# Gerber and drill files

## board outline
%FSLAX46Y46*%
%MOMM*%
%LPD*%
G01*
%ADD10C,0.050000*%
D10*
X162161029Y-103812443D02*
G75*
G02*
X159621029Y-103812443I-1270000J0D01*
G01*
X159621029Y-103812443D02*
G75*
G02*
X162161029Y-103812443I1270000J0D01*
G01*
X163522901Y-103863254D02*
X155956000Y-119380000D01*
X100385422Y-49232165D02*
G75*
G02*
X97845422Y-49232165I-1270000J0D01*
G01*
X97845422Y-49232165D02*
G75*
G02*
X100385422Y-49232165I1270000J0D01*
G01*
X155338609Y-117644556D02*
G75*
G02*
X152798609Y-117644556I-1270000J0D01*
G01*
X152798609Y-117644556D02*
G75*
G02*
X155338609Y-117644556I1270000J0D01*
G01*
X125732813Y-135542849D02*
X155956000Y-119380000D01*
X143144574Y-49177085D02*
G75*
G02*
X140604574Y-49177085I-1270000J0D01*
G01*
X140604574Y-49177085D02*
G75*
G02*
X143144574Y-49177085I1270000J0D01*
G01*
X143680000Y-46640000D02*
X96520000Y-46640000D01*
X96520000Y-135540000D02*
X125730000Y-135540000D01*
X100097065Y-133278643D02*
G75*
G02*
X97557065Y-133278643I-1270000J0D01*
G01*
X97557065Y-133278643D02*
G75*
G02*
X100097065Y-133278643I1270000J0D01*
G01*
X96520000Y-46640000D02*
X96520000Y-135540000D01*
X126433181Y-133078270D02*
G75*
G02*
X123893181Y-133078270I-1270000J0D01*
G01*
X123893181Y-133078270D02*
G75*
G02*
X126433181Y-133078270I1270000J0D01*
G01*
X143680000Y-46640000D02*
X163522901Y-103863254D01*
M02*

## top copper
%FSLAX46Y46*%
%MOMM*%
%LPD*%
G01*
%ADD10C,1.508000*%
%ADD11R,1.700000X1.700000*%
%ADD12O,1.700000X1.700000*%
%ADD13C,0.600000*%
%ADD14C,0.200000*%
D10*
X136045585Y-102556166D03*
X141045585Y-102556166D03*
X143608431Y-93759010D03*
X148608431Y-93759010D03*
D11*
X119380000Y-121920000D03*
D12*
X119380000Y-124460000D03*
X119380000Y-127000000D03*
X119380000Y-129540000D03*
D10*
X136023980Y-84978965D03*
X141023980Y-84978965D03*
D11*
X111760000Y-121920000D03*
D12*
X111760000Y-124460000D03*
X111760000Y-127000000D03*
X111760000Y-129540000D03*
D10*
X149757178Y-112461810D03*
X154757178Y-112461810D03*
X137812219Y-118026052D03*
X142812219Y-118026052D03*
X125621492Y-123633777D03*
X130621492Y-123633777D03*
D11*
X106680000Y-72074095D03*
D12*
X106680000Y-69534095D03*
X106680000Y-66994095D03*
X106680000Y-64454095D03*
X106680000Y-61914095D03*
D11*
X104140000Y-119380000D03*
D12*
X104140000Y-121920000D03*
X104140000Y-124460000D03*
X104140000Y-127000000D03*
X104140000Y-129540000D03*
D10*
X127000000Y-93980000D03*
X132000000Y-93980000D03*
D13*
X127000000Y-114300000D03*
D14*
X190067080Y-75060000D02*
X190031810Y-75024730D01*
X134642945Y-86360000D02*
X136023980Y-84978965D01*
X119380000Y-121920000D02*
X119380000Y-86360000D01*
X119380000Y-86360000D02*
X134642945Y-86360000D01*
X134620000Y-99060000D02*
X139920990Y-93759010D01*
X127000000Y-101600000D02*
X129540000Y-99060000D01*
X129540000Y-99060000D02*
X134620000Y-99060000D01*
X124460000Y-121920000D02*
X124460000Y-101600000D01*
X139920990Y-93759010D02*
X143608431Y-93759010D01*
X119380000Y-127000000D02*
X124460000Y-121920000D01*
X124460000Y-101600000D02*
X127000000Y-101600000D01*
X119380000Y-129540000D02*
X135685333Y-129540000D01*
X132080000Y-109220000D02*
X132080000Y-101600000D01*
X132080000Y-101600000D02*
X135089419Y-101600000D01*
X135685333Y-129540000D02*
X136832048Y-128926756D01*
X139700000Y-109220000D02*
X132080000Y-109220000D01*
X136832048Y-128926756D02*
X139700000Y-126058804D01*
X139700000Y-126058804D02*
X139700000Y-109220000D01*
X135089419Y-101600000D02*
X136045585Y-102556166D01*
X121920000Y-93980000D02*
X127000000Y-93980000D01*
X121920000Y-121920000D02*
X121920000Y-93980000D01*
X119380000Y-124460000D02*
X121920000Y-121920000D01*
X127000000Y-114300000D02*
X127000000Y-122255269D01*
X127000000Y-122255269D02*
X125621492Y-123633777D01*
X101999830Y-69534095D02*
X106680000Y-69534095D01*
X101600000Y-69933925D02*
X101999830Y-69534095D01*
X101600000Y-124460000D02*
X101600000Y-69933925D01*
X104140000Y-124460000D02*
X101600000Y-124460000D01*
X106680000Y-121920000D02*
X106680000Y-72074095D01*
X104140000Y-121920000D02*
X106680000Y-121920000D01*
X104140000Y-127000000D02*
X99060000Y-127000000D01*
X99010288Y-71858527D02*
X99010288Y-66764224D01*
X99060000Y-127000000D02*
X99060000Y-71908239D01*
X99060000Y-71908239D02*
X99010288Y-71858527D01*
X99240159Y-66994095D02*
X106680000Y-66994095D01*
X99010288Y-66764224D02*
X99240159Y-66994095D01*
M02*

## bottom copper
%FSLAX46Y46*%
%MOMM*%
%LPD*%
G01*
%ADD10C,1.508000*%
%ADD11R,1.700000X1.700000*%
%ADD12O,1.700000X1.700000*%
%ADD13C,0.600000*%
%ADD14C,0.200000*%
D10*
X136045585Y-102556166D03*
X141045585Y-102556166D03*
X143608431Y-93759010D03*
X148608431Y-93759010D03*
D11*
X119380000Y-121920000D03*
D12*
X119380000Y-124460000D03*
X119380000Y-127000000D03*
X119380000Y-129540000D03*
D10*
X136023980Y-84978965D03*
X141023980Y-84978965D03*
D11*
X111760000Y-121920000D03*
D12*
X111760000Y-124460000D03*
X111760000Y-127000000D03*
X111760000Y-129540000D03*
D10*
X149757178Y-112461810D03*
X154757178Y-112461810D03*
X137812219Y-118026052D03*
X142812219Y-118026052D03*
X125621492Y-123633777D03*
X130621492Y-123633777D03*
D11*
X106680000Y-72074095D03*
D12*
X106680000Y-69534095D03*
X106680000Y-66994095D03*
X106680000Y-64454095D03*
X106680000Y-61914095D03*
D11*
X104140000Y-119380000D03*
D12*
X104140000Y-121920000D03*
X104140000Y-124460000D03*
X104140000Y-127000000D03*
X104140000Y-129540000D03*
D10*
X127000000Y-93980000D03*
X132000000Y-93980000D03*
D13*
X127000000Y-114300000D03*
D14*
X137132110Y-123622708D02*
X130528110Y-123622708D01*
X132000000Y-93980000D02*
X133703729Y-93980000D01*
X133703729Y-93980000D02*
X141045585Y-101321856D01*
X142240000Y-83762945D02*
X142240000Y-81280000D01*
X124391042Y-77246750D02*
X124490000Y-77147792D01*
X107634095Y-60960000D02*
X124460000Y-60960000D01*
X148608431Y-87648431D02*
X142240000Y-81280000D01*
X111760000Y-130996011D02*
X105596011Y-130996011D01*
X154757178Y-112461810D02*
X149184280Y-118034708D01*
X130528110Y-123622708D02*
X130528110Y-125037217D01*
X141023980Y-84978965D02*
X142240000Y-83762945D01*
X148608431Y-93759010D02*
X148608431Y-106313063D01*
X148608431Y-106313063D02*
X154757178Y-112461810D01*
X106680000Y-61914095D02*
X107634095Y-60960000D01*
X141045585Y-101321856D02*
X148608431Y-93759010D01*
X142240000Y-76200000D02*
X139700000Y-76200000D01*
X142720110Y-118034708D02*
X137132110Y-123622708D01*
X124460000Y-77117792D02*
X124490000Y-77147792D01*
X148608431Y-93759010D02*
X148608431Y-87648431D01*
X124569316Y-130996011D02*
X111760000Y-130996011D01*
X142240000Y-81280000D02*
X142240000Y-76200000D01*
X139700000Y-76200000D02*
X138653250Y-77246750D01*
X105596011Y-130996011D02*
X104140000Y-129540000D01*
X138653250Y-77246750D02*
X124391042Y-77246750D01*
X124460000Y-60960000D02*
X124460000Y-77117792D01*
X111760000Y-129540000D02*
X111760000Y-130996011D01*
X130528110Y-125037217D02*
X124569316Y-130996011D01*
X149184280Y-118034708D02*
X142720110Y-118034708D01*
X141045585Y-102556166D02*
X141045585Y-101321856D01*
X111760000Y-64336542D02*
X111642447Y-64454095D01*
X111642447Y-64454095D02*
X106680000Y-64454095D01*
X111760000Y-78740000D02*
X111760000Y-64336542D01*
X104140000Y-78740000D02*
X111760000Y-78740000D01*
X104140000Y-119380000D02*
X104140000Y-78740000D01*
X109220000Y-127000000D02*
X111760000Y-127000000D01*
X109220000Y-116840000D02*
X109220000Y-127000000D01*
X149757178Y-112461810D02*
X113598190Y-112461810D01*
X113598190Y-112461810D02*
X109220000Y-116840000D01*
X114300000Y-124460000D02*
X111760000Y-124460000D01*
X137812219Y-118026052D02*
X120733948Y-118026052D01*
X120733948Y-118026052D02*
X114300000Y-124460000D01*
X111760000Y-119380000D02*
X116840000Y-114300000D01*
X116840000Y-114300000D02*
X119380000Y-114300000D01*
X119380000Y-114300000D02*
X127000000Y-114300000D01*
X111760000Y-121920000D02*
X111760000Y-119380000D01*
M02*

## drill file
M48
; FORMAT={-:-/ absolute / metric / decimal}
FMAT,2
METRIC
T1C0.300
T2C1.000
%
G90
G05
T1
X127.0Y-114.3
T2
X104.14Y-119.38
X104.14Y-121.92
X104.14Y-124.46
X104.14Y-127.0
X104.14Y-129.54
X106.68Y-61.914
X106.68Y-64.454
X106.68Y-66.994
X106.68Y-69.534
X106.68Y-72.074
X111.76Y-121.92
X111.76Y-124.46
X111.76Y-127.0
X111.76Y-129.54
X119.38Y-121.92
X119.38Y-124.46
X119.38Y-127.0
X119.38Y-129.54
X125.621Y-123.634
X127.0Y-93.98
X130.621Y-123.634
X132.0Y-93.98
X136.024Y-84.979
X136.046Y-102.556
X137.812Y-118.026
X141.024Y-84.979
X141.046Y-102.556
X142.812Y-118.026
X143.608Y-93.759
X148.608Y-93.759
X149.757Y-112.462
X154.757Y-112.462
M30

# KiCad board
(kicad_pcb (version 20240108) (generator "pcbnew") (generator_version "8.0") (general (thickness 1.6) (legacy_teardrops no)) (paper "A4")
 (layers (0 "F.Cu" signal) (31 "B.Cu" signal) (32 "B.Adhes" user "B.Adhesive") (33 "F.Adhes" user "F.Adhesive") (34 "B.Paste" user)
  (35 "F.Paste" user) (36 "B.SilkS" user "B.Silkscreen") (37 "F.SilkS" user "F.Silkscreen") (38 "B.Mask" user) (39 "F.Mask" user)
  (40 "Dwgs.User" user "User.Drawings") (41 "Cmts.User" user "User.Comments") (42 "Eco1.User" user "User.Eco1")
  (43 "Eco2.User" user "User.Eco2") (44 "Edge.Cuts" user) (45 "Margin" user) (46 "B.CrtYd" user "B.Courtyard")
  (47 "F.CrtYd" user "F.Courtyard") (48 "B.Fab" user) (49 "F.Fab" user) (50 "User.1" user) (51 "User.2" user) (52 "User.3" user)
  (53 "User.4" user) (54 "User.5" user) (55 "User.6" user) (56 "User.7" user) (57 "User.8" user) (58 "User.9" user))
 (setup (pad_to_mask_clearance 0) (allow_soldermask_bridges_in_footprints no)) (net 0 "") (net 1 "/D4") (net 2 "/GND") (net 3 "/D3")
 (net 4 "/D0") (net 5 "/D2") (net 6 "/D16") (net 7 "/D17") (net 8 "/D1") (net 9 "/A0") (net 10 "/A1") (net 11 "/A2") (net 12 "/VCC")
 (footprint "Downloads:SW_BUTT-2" (layer "F.Cu") (at 138.545585 102.556166)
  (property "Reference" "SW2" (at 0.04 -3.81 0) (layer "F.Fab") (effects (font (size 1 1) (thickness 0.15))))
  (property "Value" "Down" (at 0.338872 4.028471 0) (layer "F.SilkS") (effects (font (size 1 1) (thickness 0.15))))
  (pad "1" thru_hole circle (at -2.5 0) (size 1.508 1.508) (drill 1) (layers "*.Cu" "*.Mask") (remove_unused_layers no) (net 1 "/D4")
   (solder_mask_margin 0.102))
  (pad "2" thru_hole circle (at 2.5 0) (size 1.508 1.508) (drill 1) (layers "*.Cu" "*.Mask") (remove_unused_layers no) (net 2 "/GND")
   (solder_mask_margin 0.102)))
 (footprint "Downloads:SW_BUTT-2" (layer "F.Cu") (at 146.108431 93.75901)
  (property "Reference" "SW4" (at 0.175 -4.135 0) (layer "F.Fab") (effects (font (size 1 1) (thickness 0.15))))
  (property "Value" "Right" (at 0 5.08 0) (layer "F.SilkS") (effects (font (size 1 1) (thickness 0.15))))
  (pad "1" thru_hole circle (at -2.5 0) (size 1.508 1.508) (drill 1) (layers "*.Cu" "*.Mask") (remove_unused_layers no) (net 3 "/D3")
   (solder_mask_margin 0.102))
  (pad "2" thru_hole circle (at 2.5 0) (size 1.508 1.508) (drill 1) (layers "*.Cu" "*.Mask") (remove_unused_layers no) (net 2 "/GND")
   (solder_mask_margin 0.102)))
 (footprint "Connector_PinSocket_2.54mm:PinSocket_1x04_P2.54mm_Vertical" (layer "F.Cu") (at 119.38 121.92)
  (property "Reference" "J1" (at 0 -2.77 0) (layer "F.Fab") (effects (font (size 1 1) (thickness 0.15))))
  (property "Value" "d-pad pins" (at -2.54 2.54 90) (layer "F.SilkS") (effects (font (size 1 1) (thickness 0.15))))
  (pad "1" thru_hole rect (at 0 0) (size 1.7 1.7) (drill 1) (layers "*.Cu" "*.Mask") (remove_unused_layers no) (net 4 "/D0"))
  (pad "2" thru_hole oval (at 0 2.54) (size 1.7 1.7) (drill 1) (layers "*.Cu" "*.Mask") (remove_unused_layers no) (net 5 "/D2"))
  (pad "3" thru_hole oval (at 0 5.08) (size 1.7 1.7) (drill 1) (layers "*.Cu" "*.Mask") (remove_unused_layers no) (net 3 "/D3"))
  (pad "4" thru_hole oval (at 0 7.62) (size 1.7 1.7) (drill 1) (layers "*.Cu" "*.Mask") (remove_unused_layers no) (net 1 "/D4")))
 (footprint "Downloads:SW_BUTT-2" (layer "F.Cu") (at 138.52398 84.978965)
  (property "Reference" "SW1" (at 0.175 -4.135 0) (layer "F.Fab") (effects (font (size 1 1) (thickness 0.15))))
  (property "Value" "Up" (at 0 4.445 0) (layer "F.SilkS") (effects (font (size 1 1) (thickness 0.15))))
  (pad "1" thru_hole circle (at -2.5 0) (size 1.508 1.508) (drill 1) (layers "*.Cu" "*.Mask") (remove_unused_layers no) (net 4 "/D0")
   (solder_mask_margin 0.102))
  (pad "2" thru_hole circle (at 2.5 0) (size 1.508 1.508) (drill 1) (layers "*.Cu" "*.Mask") (remove_unused_layers no) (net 2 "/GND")
   (solder_mask_margin 0.102)))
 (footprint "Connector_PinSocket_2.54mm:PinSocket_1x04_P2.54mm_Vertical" (layer "F.Cu") (at 111.76 121.92)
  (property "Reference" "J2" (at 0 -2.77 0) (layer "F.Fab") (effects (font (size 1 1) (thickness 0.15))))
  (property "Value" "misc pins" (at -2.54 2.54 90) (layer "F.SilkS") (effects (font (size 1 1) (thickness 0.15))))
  (pad "1" thru_hole rect (at 0 0) (size 1.7 1.7) (drill 1) (layers "*.Cu" "*.Mask") (remove_unused_layers no) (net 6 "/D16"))
  (pad "2" thru_hole oval (at 0 2.54) (size 1.7 1.7) (drill 1) (layers "*.Cu" "*.Mask") (remove_unused_layers no) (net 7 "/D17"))
  (pad "3" thru_hole oval (at 0 5.08) (size 1.7 1.7) (drill 1) (layers "*.Cu" "*.Mask") (remove_unused_layers no) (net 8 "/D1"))
  (pad "4" thru_hole oval (at 0 7.62) (size 1.7 1.7) (drill 1) (layers "*.Cu" "*.Mask") (remove_unused_layers no) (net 2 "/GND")))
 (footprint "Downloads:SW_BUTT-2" (layer "F.Cu") (at 152.257178 112.46181)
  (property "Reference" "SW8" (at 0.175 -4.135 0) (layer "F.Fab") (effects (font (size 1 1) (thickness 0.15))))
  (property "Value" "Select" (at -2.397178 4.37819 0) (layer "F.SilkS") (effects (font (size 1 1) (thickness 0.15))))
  (pad "1" thru_hole circle (at -2.5 0) (size 1.508 1.508) (drill 1) (layers "*.Cu" "*.Mask") (remove_unused_layers no) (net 8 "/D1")
   (solder_mask_margin 0.102))
  (pad "2" thru_hole circle (at 2.5 0) (size 1.508 1.508) (drill 1) (layers "*.Cu" "*.Mask") (remove_unused_layers no) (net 2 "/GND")
   (solder_mask_margin 0.102)))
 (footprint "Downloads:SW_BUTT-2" (layer "F.Cu") (at 140.312219 118.026052)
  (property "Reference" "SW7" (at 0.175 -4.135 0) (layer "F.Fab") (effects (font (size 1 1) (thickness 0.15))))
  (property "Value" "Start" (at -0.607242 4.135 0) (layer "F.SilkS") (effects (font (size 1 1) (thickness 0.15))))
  (pad "1" thru_hole circle (at -2.5 0) (size 1.508 1.508) (drill 1) (layers "*.Cu" "*.Mask") (remove_unused_layers no) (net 7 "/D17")
   (solder_mask_margin 0.102))
  (pad "2" thru_hole circle (at 2.5 0) (size 1.508 1.508) (drill 1) (layers "*.Cu" "*.Mask") (remove_unused_layers no) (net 2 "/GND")
   (solder_mask_margin 0.102)))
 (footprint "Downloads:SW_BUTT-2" (layer "F.Cu") (at 128.121492 123.633777)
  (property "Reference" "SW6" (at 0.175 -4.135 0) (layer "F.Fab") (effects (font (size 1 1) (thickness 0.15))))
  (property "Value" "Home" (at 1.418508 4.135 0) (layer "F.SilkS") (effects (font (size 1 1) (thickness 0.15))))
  (pad "1" thru_hole circle (at -2.5 0) (size 1.508 1.508) (drill 1) (layers "*.Cu" "*.Mask") (remove_unused_layers no) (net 6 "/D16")
   (solder_mask_margin 0.102))
  (pad "2" thru_hole circle (at 2.5 0) (size 1.508 1.508) (drill 1) (layers "*.Cu" "*.Mask") (remove_unused_layers no) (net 2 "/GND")
   (solder_mask_margin 0.102)))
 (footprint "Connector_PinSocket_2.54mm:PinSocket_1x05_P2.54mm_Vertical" (layer "F.Cu") (at 106.68 72.074095 180)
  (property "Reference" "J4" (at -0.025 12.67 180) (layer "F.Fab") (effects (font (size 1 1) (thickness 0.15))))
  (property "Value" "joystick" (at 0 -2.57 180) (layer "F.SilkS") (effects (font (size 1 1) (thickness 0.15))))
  (pad "1" thru_hole rect (at 0 0 180) (size 1.7 1.7) (drill 1) (layers "*.Cu" "*.Mask") (remove_unused_layers no) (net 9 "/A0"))
  (pad "2" thru_hole oval (at 0 2.54 180) (size 1.7 1.7) (drill 1) (layers "*.Cu" "*.Mask") (remove_unused_layers no) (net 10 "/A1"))
  (pad "3" thru_hole oval (at 0 5.08 180) (size 1.7 1.7) (drill 1) (layers "*.Cu" "*.Mask") (remove_unused_layers no) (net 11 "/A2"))
  (pad "4" thru_hole oval (at 0 7.62 180) (size 1.7 1.7) (drill 1) (layers "*.Cu" "*.Mask") (remove_unused_layers no) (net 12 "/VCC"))
  (pad "5" thru_hole oval (at 0 10.16 180) (size 1.7 1.7) (drill 1) (layers "*.Cu" "*.Mask") (remove_unused_layers no) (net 2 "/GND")))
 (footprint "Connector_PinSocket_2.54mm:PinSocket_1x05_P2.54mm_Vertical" (layer "F.Cu") (at 104.14 119.38)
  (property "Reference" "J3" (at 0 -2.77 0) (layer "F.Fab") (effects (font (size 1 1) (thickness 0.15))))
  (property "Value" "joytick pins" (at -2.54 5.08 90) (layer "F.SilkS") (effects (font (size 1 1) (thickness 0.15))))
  (pad "1" thru_hole rect (at 0 0) (size 1.7 1.7) (drill 1) (layers "*.Cu" "*.Mask") (remove_unused_layers no) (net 12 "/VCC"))
  (pad "2" thru_hole oval (at 0 2.54) (size 1.7 1.7) (drill 1) (layers "*.Cu" "*.Mask") (remove_unused_layers no) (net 9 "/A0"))
  (pad "3" thru_hole oval (at 0 5.08) (size 1.7 1.7) (drill 1) (layers "*.Cu" "*.Mask") (remove_unused_layers no) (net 10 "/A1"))
  (pad "4" thru_hole oval (at 0 7.62) (size 1.7 1.7) (drill 1) (layers "*.Cu" "*.Mask") (remove_unused_layers no) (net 11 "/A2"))
  (pad "5" thru_hole oval (at 0 10.16) (size 1.7 1.7) (drill 1) (layers "*.Cu" "*.Mask") (remove_unused_layers no) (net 2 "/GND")))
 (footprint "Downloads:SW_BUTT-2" (layer "F.Cu") (at 129.5 93.98)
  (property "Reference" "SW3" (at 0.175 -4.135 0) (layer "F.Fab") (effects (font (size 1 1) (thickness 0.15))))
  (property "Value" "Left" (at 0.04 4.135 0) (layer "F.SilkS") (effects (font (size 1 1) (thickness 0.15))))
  (pad "1" thru_hole circle (at -2.5 0) (size 1.508 1.508) (drill 1) (layers "*.Cu" "*.Mask") (remove_unused_layers no) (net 5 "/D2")
   (solder_mask_margin 0.102))
  (pad "2" thru_hole circle (at 2.5 0) (size 1.508 1.508) (drill 1) (layers "*.Cu" "*.Mask") (remove_unused_layers no) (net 2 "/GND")
   (solder_mask_margin 0.102)))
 (gr_circle (center 160.891029 103.812443) (end 162.161029 103.812443) (stroke (width 0.05) (type default)) (fill none) (layer "Edge.Cuts"))
 (gr_line (start 163.522901 103.863254) (end 155.956 119.38) (stroke (width 0.05) (type default)) (layer "Edge.Cuts"))
 (gr_circle (center 99.115422 49.232165) (end 97.845422 49.232165) (stroke (width 0.05) (type default)) (fill none) (layer "Edge.Cuts"))
 (gr_circle (center 154.068609 117.644556) (end 155.338609 117.644556) (stroke (width 0.05) (type default)) (fill none) (layer "Edge.Cuts"))
 (gr_line (start 125.732813 135.542849) (end 155.956 119.38) (stroke (width 0.05) (type default)) (layer "Edge.Cuts"))
 (gr_circle (center 141.874574 49.177085) (end 141.874574 47.907085) (stroke (width 0.05) (type default)) (fill none) (layer "Edge.Cuts"))
 (gr_line (start 143.68 46.64) (end 96.52 46.64) (stroke (width 0.05) (type default)) (layer "Edge.Cuts"))
 (gr_line (start 96.52 135.54) (end 125.73 135.54) (stroke (width 0.05) (type default)) (layer "Edge.Cuts"))
 (gr_circle (center 98.827065 133.278643) (end 100.097065 133.278643) (stroke (width 0.05) (type default)) (fill none) (layer "Edge.Cuts"))
 (gr_line (start 96.52 46.64) (end 96.52 135.54) (stroke (width 0.05) (type default)) (layer "Edge.Cuts"))
 (gr_circle (center 125.163181 133.07827) (end 126.433181 133.07827) (stroke (width 0.05) (type default)) (fill none) (layer "Edge.Cuts"))
 (gr_line (start 143.68 46.64) (end 163.522901 103.863254) (stroke (width 0.05) (type default)) (layer "Edge.Cuts"))
 (segment (start 190.06708 75.06) (end 190.03181 75.02473) (width 0.2) (layer "F.Cu") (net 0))
 (segment (start 137.13211 123.622708) (end 130.52811 123.622708) (width 0.2) (layer "B.Cu") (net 2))
 (segment (start 132 93.98) (end 133.703729 93.98) (width 0.2) (layer "B.Cu") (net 2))
 (segment (start 133.703729 93.98) (end 141.045585 101.321856) (width 0.2) (layer "B.Cu") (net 2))
 (segment (start 142.24 83.762945) (end 142.24 81.28) (width 0.2) (layer "B.Cu") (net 2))
 (segment (start 124.391042 77.24675) (end 124.49 77.147792) (width 0.2) (layer "B.Cu") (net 2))
 (segment (start 107.634095 60.96) (end 124.46 60.96) (width 0.2) (layer "B.Cu") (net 2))
 (segment (start 148.608431 87.648431) (end 142.24 81.28) (width 0.2) (layer "B.Cu") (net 2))
 (segment (start 111.76 130.996011) (end 105.596011 130.996011) (width 0.2) (layer "B.Cu") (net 2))
 (segment (start 154.757178 112.46181) (end 149.18428 118.034708) (width 0.2) (layer "B.Cu") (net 2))
 (segment (start 130.52811 123.622708) (end 130.52811 125.037217) (width 0.2) (layer "B.Cu") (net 2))
 (segment (start 141.02398 84.978965) (end 142.24 83.762945) (width 0.2) (layer "B.Cu") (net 2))
 (segment (start 148.608431 93.75901) (end 148.608431 106.313063) (width 0.2) (layer "B.Cu") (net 2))
 (segment (start 148.608431 106.313063) (end 154.757178 112.46181) (width 0.2) (layer "B.Cu") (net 2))
 (segment (start 106.68 61.914095) (end 107.634095 60.96) (width 0.2) (layer "B.Cu") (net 2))
 (segment (start 141.045585 101.321856) (end 148.608431 93.75901) (width 0.2) (layer "B.Cu") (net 2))
 (segment (start 142.24 76.2) (end 139.7 76.2) (width 0.2) (layer "B.Cu") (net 2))
 (segment (start 142.72011 118.034708) (end 137.13211 123.622708) (width 0.2) (layer "B.Cu") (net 2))
 (segment (start 124.46 77.117792) (end 124.49 77.147792) (width 0.2) (layer "B.Cu") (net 2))
 (segment (start 148.608431 93.75901) (end 148.608431 87.648431) (width 0.2) (layer "B.Cu") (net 2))
 (segment (start 124.569316 130.996011) (end 111.76 130.996011) (width 0.2) (layer "B.Cu") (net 2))
 (segment (start 142.24 81.28) (end 142.24 76.2) (width 0.2) (layer "B.Cu") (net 2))
 (segment (start 139.7 76.2) (end 138.65325 77.24675) (width 0.2) (layer "B.Cu") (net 2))
 (segment (start 105.596011 130.996011) (end 104.14 129.54) (width 0.2) (layer "B.Cu") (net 2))
 (segment (start 138.65325 77.24675) (end 124.391042 77.24675) (width 0.2) (layer "B.Cu") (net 2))
 (segment (start 124.46 60.96) (end 124.46 77.117792) (width 0.2) (layer "B.Cu") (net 2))
 (segment (start 111.76 129.54) (end 111.76 130.996011) (width 0.2) (layer "B.Cu") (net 2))
 (segment (start 130.52811 125.037217) (end 124.569316 130.996011) (width 0.2) (layer "B.Cu") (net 2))
 (segment (start 149.18428 118.034708) (end 142.72011 118.034708) (width 0.2) (layer "B.Cu") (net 2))
 (segment (start 141.045585 102.556166) (end 141.045585 101.321856) (width 0.2) (layer "B.Cu") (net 2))
 (segment (start 111.76 64.336542) (end 111.642447 64.454095) (width 0.2) (layer "B.Cu") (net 12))
 (segment (start 111.642447 64.454095) (end 106.68 64.454095) (width 0.2) (layer "B.Cu") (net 12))
 (segment (start 111.76 78.74) (end 111.76 64.336542) (width 0.2) (layer "B.Cu") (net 12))
 (segment (start 104.14 78.74) (end 111.76 78.74) (width 0.2) (layer "B.Cu") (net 12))
 (segment (start 104.14 119.38) (end 104.14 78.74) (width 0.2) (layer "B.Cu") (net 12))
 (segment (start 134.642945 86.36) (end 136.02398 84.978965) (width 0.2) (layer "F.Cu") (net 4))
 (segment (start 119.38 121.92) (end 119.38 86.36) (width 0.2) (layer "F.Cu") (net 4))
 (segment (start 119.38 86.36) (end 134.642945 86.36) (width 0.2) (layer "F.Cu") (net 4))
 (segment (start 134.62 99.06) (end 139.92099 93.75901) (width 0.2) (layer "F.Cu") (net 3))
 (segment (start 127 101.6) (end 129.54 99.06) (width 0.2) (layer "F.Cu") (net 3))
 (segment (start 129.54 99.06) (end 134.62 99.06) (width 0.2) (layer "F.Cu") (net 3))
 (segment (start 124.46 121.92) (end 124.46 101.6) (width 0.2) (layer "F.Cu") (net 3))
 (segment (start 139.92099 93.75901) (end 143.608431 93.75901) (width 0.2) (layer "F.Cu") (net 3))
 (segment (start 119.38 127) (end 124.46 121.92) (width 0.2) (layer "F.Cu") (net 3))
 (segment (start 124.46 101.6) (end 127 101.6) (width 0.2) (layer "F.Cu") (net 3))
 (segment (start 119.38 129.54) (end 135.685333 129.54) (width 0.2) (layer "F.Cu") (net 1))
 (segment (start 132.08 109.22) (end 132.08 101.6) (width 0.2) (layer "F.Cu") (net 1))
 (segment (start 132.08 101.6) (end 135.089419 101.6) (width 0.2) (layer "F.Cu") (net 1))
 (segment (start 135.685333 129.54) (end 136.832048 128.926756) (width 0.2) (layer "F.Cu") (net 1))
 (segment (start 139.7 109.22) (end 132.08 109.22) (width 0.2) (layer "F.Cu") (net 1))
 (segment (start 136.832048 128.926756) (end 139.7 126.058804) (width 0.2) (layer "F.Cu") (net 1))
 (segment (start 139.7 126.058804) (end 139.7 109.22) (width 0.2) (layer "F.Cu") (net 1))
 (segment (start 135.089419 101.6) (end 136.045585 102.556166) (width 0.2) (layer "F.Cu") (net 1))
 (segment (start 121.92 93.98) (end 127 93.98) (width 0.2) (layer "F.Cu") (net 5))
 (segment (start 121.92 121.92) (end 121.92 93.98) (width 0.2) (layer "F.Cu") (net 5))
 (segment (start 119.38 124.46) (end 121.92 121.92) (width 0.2) (layer "F.Cu") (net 5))
 (segment (start 109.22 127) (end 111.76 127) (width 0.2) (layer "B.Cu") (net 8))
 (segment (start 109.22 116.84) (end 109.22 127) (width 0.2) (layer "B.Cu") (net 8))
 (segment (start 149.757178 112.46181) (end 113.59819 112.46181) (width 0.2) (layer "B.Cu") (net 8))
 (segment (start 113.59819 112.46181) (end 109.22 116.84) (width 0.2) (layer "B.Cu") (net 8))
 (segment (start 114.3 124.46) (end 111.76 124.46) (width 0.2) (layer "B.Cu") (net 7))
 (segment (start 137.812219 118.026052) (end 120.733948 118.026052) (width 0.2) (layer "B.Cu") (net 7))
 (segment (start 120.733948 118.026052) (end 114.3 124.46) (width 0.2) (layer "B.Cu") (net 7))
 (segment (start 127 114.3) (end 127 122.255269) (width 0.2) (layer "F.Cu") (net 6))
 (segment (start 127 122.255269) (end 125.621492 123.633777) (width 0.2) (layer "F.Cu") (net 6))
 (via (at 127 114.3) (size 0.6) (drill 0.3) (layers "F.Cu" "B.Cu") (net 6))
 (segment (start 111.76 119.38) (end 116.84 114.3) (width 0.2) (layer "B.Cu") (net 6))
 (segment (start 116.84 114.3) (end 119.38 114.3) (width 0.2) (layer "B.Cu") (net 6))
 (segment (start 119.38 114.3) (end 127 114.3) (width 0.2) (layer "B.Cu") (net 6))
 (segment (start 111.76 121.92) (end 111.76 119.38) (width 0.2) (layer "B.Cu") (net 6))
 (segment (start 101.99983 69.534095) (end 106.68 69.534095) (width 0.2) (layer "F.Cu") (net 10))
 (segment (start 101.6 69.933925) (end 101.99983 69.534095) (width 0.2) (layer "F.Cu") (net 10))
 (segment (start 101.6 124.46) (end 101.6 69.933925) (width 0.2) (layer "F.Cu") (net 10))
 (segment (start 104.14 124.46) (end 101.6 124.46) (width 0.2) (layer "F.Cu") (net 10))
 (segment (start 106.68 121.92) (end 106.68 72.074095) (width 0.2) (layer "F.Cu") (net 9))
 (segment (start 104.14 121.92) (end 106.68 121.92) (width 0.2) (layer "F.Cu") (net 9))
 (segment (start 104.14 127) (end 99.06 127) (width 0.2) (layer "F.Cu") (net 11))
 (segment (start 99.010288 71.858527) (end 99.010288 66.764224) (width 0.2) (layer "F.Cu") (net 11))
 (segment (start 99.06 127) (end 99.06 71.908239) (width 0.2) (layer "F.Cu") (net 11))
 (segment (start 99.06 71.908239) (end 99.010288 71.858527) (width 0.2) (layer "F.Cu") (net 11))
 (segment (start 99.240159 66.994095) (end 106.68 66.994095) (width 0.2) (layer "F.Cu") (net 11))
 (segment (start 99.010288 66.764224) (end 99.240159 66.994095) (width 0.2) (layer "F.Cu") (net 11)))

